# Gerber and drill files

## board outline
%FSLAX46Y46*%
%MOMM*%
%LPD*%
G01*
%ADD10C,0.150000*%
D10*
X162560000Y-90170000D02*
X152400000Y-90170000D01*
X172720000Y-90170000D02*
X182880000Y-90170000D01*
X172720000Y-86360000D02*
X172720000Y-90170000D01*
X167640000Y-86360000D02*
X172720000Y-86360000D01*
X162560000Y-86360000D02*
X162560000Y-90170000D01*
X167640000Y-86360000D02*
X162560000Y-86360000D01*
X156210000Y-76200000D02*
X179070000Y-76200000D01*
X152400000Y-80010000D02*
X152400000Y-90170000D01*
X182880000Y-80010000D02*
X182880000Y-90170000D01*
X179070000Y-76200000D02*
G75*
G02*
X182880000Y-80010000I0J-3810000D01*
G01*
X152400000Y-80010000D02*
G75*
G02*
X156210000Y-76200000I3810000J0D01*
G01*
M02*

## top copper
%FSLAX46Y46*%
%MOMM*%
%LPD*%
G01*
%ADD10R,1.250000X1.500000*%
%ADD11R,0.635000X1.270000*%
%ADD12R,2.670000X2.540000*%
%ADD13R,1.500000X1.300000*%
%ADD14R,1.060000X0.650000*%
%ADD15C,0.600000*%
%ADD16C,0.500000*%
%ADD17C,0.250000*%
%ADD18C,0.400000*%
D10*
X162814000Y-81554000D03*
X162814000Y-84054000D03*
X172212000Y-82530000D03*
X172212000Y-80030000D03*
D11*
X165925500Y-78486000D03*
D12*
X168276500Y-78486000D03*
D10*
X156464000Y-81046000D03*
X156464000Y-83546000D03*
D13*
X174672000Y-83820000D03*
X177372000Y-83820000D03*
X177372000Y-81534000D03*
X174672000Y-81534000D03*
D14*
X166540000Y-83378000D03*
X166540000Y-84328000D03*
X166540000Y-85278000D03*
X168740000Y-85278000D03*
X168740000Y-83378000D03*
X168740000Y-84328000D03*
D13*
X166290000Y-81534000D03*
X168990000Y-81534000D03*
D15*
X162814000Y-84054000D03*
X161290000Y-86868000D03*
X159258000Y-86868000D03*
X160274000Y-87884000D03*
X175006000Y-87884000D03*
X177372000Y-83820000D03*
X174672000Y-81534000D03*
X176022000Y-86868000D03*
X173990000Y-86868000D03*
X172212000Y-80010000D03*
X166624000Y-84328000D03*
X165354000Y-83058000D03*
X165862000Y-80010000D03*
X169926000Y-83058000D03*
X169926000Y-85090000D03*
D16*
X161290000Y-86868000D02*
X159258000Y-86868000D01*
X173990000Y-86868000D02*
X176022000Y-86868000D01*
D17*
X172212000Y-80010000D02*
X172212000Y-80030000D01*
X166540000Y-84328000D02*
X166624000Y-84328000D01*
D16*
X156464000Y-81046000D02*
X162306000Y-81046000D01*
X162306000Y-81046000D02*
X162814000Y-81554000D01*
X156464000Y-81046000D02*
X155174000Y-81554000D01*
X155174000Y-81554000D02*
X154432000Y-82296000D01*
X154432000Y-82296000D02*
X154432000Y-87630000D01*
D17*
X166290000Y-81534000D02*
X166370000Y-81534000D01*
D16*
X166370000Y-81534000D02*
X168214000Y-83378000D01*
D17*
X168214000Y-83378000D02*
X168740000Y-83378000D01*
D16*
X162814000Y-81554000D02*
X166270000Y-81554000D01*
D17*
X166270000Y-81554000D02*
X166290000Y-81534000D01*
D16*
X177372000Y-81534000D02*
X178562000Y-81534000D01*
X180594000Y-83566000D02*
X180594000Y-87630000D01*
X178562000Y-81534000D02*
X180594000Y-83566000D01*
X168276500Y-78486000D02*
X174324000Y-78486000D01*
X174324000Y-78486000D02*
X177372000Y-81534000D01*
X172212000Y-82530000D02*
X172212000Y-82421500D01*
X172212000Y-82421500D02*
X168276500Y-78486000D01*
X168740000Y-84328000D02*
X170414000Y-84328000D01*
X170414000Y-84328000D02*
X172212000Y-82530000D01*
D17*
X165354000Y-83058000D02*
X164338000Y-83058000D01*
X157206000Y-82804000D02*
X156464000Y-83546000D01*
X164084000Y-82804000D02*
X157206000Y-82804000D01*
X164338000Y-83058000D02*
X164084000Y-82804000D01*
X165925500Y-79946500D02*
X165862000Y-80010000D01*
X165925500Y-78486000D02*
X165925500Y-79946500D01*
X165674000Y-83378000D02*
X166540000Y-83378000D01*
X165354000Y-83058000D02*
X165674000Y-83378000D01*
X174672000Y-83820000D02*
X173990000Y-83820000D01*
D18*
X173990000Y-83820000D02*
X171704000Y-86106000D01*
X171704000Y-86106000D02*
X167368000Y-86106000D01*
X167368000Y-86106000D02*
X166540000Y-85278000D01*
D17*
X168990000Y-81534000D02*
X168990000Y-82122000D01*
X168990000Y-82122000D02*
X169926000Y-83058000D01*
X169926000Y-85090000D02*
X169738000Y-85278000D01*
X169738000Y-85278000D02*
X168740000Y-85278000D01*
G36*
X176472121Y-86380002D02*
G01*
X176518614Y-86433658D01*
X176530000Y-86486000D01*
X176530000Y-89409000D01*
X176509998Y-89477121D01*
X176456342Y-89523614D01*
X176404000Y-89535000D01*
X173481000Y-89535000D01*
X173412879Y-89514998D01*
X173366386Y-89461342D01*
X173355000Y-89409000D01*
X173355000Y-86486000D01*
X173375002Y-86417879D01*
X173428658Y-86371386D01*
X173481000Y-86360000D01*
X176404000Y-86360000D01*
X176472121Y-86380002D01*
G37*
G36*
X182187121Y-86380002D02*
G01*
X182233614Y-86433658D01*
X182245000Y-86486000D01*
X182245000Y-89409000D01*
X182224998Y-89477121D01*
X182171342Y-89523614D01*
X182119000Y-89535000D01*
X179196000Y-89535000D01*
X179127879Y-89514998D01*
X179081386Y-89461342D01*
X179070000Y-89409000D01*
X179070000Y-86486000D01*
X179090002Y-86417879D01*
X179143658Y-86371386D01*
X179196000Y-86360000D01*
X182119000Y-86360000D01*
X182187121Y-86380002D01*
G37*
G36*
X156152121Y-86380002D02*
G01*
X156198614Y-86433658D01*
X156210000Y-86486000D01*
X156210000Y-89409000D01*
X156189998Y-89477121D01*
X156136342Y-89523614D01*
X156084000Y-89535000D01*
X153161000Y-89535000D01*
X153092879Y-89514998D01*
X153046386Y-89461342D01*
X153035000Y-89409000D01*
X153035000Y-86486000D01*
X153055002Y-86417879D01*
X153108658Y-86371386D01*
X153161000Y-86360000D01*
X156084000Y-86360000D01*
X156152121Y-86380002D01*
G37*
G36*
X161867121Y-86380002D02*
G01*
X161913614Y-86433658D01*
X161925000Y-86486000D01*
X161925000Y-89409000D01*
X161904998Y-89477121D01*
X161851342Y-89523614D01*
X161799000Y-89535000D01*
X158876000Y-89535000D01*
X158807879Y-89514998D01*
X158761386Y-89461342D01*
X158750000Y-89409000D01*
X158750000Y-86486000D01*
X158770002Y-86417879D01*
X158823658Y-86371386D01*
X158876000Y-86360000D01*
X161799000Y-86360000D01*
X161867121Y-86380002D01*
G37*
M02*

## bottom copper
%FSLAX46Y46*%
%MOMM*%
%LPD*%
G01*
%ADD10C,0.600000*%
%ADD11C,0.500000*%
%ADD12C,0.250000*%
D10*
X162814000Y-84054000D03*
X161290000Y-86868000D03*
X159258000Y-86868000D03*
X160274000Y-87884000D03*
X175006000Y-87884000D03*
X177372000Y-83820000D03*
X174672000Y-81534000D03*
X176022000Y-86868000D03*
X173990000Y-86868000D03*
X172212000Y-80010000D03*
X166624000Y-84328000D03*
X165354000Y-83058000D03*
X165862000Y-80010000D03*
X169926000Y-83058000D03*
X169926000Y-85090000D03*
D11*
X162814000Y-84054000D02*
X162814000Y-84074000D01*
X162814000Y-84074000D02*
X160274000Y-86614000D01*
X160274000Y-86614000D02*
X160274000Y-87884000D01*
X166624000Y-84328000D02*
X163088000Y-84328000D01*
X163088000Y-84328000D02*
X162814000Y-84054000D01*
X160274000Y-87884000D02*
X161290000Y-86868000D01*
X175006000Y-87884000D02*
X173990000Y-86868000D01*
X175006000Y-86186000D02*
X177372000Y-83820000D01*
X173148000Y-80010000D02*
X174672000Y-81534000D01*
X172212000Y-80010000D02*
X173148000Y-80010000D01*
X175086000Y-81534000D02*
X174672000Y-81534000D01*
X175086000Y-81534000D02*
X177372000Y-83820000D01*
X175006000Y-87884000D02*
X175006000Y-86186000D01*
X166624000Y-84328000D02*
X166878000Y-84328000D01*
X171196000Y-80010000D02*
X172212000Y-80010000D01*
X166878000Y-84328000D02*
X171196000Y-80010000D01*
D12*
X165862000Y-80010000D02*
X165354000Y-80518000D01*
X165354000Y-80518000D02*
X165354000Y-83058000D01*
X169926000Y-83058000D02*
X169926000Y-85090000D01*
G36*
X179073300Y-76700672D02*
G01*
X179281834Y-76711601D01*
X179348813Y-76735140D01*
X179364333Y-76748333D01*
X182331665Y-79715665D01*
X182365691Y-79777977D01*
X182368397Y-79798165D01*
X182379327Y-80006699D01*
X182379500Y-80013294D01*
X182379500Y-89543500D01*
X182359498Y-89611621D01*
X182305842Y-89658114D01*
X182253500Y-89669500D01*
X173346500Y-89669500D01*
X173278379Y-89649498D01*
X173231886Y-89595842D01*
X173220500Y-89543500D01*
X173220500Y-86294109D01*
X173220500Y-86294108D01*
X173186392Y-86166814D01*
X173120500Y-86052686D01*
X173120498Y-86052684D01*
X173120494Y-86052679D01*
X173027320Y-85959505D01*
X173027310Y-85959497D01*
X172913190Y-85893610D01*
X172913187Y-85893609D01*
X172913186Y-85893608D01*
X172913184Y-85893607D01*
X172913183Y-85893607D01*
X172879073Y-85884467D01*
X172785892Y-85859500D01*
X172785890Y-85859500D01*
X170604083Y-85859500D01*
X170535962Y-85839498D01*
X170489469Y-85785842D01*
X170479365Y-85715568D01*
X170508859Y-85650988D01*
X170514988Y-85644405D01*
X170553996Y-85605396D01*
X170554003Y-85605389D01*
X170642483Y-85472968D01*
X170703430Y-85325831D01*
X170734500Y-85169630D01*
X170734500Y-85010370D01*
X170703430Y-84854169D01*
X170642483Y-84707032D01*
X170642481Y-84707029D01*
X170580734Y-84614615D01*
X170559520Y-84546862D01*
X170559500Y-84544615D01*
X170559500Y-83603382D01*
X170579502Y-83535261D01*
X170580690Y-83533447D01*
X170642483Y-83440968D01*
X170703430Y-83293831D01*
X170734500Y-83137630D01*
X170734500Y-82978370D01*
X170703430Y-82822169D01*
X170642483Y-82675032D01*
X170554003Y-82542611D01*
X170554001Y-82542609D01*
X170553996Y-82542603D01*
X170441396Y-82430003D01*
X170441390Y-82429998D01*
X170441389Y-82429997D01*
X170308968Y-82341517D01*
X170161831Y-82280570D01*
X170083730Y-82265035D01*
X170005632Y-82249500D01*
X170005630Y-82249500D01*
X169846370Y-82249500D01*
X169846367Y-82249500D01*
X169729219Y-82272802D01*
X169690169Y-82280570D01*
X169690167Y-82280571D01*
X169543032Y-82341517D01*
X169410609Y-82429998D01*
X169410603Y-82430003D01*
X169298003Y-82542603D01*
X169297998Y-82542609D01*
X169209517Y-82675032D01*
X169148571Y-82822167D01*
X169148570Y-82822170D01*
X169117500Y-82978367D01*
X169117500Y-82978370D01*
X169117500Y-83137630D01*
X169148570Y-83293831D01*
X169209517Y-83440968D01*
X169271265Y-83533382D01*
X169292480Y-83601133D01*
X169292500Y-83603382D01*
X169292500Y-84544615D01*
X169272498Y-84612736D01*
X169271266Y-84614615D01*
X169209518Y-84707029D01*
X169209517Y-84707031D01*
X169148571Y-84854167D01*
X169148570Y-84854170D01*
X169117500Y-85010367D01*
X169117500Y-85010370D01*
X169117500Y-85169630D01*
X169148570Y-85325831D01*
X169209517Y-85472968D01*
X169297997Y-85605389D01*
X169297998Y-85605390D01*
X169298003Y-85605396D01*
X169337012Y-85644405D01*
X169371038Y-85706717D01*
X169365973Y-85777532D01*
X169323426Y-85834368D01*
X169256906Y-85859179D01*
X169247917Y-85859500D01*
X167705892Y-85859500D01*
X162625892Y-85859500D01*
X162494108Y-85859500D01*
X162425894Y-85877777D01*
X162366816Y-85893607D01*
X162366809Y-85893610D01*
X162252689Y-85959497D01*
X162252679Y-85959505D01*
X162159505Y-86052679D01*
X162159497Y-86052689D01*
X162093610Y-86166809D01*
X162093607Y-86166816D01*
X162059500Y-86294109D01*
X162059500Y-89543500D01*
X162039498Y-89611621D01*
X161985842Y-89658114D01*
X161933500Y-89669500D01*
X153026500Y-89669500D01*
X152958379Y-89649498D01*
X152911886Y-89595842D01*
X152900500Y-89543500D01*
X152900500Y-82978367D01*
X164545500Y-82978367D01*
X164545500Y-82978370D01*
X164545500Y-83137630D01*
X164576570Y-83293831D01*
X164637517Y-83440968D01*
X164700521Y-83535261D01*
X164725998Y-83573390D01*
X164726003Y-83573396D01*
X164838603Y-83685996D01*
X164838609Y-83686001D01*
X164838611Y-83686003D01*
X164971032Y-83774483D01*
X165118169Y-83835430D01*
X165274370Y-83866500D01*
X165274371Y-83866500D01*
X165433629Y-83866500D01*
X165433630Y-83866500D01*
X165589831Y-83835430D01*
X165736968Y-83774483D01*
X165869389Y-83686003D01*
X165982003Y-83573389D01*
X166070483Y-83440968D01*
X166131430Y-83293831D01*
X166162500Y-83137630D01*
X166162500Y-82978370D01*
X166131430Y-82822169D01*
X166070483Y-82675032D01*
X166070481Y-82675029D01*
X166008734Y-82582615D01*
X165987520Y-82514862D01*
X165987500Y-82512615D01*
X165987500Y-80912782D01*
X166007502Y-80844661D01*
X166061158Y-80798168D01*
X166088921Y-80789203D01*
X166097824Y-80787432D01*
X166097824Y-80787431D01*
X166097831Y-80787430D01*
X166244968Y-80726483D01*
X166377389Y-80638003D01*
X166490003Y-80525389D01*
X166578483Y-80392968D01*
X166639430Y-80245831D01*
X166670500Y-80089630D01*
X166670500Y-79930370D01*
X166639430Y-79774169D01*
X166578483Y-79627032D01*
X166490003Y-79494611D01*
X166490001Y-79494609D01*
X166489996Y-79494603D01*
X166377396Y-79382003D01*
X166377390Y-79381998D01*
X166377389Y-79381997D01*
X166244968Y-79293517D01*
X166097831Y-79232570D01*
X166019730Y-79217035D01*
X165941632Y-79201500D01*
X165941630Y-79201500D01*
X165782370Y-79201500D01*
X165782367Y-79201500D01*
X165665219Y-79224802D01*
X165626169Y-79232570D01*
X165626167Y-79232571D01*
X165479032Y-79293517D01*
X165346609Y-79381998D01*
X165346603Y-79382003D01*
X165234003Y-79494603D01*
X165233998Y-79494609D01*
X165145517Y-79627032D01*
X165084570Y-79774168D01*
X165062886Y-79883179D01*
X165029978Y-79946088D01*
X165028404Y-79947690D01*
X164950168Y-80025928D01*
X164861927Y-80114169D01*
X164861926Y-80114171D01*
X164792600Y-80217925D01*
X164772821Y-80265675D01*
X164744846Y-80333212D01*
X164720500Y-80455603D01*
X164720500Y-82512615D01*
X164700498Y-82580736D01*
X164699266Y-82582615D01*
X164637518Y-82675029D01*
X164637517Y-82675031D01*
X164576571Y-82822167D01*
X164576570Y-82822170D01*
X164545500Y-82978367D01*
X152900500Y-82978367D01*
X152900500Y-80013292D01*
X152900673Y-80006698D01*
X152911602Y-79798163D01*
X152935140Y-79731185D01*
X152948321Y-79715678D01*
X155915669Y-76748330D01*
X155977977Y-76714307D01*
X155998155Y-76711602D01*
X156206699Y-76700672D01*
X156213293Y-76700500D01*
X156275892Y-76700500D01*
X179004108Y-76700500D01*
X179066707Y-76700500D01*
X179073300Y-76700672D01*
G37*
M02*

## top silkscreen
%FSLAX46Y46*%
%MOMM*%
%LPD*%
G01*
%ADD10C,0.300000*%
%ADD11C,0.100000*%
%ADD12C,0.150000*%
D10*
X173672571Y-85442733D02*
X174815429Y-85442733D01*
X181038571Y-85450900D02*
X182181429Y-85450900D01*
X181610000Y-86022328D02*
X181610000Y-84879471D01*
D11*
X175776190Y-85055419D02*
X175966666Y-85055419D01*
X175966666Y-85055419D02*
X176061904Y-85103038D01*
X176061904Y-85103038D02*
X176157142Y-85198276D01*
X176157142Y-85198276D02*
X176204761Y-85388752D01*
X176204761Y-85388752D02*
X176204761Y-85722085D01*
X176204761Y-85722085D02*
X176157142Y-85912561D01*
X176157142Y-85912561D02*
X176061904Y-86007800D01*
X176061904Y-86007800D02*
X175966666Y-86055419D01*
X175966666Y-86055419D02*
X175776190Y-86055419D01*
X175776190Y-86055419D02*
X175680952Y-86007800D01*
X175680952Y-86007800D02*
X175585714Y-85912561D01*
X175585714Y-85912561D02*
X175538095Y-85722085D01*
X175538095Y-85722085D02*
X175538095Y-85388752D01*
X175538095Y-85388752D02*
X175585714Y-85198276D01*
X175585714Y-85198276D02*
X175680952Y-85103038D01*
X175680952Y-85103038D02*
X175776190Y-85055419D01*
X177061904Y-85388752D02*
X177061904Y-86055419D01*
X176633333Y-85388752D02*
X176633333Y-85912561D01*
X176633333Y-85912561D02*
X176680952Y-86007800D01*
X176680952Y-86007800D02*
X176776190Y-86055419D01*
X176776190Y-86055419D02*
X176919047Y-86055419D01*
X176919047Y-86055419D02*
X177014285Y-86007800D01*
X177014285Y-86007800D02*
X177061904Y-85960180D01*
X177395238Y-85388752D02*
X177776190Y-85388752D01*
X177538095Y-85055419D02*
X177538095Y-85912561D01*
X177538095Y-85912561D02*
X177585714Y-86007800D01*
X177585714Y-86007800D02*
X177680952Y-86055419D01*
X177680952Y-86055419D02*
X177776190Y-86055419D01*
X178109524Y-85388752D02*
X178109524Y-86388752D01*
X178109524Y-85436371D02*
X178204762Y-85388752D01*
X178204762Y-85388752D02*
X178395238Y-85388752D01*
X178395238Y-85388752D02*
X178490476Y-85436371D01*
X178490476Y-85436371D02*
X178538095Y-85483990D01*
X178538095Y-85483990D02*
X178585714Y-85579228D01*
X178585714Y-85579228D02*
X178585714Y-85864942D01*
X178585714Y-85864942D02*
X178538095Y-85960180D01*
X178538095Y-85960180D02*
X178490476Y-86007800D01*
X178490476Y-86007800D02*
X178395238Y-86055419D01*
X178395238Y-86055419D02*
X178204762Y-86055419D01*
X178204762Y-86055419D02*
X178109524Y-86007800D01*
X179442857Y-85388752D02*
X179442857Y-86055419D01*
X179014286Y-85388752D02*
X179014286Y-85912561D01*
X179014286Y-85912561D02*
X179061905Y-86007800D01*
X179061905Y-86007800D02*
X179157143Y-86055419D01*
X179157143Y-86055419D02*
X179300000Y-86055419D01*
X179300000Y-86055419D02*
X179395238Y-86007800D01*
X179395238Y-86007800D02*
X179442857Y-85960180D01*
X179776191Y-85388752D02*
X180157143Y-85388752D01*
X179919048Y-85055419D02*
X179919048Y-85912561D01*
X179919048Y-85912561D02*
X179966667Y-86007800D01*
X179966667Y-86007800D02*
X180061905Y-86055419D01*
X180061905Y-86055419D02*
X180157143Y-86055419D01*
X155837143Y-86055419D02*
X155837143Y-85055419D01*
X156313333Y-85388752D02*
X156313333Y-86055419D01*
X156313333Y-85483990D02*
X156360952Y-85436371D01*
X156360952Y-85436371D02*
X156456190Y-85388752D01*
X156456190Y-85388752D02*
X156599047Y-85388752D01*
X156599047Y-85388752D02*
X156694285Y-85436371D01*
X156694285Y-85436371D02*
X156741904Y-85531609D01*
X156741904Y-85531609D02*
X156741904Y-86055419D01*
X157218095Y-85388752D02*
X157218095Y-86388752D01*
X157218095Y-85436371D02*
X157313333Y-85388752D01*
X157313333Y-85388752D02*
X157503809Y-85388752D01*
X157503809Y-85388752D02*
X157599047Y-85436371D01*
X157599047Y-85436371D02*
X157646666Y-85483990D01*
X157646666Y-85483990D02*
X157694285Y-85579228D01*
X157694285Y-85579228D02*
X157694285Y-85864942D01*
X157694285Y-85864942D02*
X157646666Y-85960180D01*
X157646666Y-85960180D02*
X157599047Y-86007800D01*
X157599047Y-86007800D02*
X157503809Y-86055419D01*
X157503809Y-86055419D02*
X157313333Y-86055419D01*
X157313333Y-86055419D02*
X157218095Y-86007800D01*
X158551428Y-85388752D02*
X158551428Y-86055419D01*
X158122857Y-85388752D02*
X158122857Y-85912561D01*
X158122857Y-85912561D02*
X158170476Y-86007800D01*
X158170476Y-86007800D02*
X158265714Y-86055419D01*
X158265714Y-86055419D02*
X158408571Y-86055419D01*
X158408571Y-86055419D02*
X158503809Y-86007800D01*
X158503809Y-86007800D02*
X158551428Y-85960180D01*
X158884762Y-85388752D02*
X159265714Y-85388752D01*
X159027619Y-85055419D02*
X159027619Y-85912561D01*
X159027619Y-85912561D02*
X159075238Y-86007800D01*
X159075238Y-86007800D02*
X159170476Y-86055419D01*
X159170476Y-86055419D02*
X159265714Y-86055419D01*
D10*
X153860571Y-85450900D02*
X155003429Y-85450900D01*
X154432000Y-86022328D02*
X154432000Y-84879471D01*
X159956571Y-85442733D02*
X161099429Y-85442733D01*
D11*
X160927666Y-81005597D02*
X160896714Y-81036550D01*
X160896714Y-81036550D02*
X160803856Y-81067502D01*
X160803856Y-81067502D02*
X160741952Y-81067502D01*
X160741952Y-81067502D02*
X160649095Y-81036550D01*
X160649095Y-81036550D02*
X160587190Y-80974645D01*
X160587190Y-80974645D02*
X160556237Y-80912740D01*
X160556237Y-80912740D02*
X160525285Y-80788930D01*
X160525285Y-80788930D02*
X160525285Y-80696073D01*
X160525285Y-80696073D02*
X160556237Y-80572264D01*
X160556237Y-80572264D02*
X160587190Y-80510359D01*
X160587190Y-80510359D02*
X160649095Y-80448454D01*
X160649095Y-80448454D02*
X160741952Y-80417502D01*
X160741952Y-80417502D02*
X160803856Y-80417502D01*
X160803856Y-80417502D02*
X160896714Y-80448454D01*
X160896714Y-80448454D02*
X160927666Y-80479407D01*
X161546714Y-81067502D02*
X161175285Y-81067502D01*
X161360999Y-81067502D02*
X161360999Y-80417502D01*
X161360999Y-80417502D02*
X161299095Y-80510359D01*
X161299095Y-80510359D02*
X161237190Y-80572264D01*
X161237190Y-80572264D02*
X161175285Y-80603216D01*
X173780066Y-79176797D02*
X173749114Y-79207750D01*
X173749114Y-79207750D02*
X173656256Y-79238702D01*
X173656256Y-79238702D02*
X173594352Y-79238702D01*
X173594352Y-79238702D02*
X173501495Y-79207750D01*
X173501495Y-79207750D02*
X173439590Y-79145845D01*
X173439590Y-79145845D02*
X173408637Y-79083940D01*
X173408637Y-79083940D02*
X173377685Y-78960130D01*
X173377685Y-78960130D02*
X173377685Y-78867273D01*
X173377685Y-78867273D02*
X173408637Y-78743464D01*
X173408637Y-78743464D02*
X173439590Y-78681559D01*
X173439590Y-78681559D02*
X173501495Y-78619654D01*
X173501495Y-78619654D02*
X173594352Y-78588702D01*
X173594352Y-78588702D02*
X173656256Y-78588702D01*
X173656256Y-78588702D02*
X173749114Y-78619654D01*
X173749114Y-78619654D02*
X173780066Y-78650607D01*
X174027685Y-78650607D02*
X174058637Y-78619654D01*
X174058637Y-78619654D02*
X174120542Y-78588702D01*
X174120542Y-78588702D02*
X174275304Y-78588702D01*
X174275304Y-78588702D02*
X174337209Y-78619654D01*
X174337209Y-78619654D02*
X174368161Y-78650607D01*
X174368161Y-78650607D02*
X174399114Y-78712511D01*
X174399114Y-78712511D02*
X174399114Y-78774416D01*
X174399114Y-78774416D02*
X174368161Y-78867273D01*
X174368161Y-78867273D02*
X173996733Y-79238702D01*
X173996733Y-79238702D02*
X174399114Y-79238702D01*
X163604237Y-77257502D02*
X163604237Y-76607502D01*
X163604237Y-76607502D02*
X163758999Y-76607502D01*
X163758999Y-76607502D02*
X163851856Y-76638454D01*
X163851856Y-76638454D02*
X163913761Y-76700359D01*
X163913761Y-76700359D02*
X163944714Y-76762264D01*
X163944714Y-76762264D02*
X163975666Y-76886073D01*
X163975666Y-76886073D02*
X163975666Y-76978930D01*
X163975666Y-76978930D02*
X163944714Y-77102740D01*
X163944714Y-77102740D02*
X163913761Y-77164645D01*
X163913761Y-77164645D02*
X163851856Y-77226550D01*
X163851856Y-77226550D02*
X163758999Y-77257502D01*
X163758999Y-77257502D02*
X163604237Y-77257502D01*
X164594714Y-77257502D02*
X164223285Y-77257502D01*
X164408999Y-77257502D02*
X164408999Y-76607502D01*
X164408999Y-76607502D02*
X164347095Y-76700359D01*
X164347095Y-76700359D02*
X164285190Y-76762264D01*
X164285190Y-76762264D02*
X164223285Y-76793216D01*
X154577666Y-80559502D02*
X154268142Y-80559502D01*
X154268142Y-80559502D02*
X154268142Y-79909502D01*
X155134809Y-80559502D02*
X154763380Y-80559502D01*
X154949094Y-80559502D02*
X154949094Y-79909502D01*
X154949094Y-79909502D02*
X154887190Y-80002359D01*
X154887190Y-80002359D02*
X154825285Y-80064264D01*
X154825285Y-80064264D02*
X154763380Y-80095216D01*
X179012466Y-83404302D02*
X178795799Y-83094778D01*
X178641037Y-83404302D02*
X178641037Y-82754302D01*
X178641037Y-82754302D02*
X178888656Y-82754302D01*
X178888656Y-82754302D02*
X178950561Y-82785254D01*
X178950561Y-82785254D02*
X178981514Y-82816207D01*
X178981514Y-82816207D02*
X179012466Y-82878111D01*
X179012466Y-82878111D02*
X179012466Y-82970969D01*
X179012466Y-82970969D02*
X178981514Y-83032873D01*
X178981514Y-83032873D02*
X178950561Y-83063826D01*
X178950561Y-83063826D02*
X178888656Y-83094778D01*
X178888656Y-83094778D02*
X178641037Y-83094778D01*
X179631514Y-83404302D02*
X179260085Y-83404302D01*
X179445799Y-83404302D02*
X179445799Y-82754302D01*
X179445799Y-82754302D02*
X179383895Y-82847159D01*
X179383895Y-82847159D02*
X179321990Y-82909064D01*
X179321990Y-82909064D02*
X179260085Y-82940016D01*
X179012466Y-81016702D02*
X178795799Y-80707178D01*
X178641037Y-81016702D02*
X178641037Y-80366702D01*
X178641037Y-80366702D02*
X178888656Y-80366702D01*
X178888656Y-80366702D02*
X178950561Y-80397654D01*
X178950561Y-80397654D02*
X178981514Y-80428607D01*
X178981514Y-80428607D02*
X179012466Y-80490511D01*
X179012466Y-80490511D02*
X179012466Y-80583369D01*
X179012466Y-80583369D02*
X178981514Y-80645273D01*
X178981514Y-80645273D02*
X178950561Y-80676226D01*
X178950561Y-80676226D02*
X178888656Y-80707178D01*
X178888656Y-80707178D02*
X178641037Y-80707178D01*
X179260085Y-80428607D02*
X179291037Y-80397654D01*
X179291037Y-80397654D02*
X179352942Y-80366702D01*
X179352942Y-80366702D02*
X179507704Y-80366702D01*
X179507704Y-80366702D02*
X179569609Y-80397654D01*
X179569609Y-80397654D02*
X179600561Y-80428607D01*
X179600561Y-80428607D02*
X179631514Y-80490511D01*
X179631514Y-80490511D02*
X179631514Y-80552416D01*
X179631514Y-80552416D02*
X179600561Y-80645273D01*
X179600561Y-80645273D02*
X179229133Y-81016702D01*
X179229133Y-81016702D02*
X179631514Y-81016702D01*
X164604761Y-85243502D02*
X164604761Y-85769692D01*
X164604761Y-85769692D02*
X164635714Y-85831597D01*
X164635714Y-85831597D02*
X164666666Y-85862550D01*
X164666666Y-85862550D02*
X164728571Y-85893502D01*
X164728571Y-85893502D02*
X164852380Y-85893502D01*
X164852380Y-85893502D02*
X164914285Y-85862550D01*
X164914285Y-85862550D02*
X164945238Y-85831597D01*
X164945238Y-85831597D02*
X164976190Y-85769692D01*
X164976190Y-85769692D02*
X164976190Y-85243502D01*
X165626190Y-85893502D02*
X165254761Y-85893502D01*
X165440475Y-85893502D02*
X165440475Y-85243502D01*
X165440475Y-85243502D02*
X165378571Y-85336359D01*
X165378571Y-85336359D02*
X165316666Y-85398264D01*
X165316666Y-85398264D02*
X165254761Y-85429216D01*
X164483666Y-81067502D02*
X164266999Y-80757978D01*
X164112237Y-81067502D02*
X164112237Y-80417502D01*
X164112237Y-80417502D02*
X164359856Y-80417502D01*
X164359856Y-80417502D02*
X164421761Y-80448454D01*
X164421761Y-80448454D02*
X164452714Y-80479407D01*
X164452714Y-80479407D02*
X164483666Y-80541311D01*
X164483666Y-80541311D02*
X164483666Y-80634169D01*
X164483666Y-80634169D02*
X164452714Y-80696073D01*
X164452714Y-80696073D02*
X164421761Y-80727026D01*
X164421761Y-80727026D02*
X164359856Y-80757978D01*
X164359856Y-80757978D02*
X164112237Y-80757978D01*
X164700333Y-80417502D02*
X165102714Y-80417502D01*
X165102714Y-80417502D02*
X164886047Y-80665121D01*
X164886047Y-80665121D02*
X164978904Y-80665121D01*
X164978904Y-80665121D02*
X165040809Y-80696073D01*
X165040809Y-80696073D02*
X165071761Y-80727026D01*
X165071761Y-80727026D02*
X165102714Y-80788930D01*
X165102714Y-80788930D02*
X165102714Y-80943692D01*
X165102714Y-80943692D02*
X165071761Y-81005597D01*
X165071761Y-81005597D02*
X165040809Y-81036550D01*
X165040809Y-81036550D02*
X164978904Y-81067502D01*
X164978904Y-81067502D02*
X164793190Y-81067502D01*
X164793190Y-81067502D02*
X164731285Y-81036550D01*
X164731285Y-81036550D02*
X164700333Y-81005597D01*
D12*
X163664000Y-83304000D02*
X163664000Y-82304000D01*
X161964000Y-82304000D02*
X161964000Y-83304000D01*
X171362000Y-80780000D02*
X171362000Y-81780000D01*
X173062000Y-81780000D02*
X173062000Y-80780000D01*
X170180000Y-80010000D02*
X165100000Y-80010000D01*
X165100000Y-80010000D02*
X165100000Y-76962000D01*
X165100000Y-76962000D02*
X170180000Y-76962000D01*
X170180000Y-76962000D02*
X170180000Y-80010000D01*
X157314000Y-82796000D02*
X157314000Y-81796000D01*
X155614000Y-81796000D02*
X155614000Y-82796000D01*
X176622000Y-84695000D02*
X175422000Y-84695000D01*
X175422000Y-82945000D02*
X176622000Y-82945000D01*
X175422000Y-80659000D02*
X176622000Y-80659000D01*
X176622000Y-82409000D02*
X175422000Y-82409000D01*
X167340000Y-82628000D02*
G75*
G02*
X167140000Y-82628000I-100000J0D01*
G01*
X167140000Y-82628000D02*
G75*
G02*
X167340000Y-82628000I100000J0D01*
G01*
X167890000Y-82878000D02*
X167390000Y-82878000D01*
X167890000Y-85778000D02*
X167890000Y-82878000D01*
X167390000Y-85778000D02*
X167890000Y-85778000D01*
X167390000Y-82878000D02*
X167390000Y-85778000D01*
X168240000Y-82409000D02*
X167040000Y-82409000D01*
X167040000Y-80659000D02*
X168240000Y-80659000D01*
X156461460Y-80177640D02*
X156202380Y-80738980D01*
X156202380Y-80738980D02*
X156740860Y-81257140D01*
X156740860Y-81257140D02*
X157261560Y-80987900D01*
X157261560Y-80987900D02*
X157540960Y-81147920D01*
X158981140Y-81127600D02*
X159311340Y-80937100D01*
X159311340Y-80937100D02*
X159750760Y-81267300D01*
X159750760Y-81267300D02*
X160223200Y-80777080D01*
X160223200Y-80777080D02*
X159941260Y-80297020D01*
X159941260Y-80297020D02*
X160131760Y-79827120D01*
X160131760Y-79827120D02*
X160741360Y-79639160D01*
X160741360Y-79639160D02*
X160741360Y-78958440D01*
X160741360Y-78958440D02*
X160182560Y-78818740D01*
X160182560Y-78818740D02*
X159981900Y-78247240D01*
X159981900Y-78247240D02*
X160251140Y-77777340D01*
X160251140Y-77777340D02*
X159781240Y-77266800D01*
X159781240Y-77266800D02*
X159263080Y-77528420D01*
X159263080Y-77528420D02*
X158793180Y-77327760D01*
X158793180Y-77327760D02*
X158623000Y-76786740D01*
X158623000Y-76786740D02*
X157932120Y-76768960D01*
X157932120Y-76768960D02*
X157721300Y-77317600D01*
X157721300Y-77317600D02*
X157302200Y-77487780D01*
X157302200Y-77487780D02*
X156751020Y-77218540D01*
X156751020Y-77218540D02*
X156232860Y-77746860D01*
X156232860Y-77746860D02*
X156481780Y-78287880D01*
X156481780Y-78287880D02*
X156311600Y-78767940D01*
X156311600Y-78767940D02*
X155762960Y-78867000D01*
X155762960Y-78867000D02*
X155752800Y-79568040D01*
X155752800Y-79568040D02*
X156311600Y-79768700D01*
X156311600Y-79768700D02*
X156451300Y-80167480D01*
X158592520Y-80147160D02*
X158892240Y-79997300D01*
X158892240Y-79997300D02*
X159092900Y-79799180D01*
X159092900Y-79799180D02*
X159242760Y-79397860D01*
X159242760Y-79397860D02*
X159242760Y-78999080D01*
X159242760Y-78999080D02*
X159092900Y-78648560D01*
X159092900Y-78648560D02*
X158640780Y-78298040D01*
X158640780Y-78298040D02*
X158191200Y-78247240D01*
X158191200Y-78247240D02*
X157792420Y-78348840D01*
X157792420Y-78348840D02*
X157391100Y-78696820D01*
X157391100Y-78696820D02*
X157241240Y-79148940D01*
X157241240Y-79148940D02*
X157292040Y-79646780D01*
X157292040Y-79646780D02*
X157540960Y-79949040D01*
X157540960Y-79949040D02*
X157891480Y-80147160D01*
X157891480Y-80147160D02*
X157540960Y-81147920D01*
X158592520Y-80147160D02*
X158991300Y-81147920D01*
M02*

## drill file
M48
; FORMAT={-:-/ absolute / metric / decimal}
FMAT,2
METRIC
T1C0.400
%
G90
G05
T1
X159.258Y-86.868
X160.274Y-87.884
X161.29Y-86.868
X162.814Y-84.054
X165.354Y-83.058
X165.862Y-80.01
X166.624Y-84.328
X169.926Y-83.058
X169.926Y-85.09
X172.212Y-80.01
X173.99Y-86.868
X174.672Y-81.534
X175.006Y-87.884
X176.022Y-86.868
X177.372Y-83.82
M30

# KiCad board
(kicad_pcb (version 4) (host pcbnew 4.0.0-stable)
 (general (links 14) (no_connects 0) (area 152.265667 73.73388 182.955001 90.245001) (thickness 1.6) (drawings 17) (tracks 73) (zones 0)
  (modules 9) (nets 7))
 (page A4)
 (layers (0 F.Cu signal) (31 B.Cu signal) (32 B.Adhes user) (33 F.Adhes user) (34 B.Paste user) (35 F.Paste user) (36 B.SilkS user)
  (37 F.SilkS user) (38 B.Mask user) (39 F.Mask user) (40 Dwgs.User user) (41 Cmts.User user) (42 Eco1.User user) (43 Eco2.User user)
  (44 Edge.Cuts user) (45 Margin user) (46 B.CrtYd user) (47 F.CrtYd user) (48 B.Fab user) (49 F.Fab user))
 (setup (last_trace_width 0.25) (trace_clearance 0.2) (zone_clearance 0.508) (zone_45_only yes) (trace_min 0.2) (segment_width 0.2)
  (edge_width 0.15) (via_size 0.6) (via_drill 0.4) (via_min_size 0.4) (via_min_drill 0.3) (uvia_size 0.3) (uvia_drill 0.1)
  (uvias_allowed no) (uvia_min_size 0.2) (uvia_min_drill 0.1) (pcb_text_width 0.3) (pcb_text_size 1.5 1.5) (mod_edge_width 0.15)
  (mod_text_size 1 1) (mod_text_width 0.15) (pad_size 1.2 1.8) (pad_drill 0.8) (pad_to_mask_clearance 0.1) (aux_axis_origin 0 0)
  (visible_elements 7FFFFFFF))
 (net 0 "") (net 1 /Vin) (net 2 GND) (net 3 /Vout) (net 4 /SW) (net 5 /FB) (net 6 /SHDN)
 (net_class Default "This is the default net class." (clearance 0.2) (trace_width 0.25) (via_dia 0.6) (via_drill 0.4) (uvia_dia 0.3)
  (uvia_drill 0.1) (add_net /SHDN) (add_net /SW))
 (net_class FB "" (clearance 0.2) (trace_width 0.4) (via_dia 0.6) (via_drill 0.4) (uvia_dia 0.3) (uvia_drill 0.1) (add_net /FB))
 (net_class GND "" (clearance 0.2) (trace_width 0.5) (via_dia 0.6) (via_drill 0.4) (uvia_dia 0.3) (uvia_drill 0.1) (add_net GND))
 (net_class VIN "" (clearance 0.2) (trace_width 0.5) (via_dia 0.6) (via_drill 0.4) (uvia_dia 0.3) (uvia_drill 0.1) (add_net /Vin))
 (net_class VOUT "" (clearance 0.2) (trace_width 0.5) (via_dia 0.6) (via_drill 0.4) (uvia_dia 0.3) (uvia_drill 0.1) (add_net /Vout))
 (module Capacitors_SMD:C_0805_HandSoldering (layer F.Cu) (at 162.814 82.804 270)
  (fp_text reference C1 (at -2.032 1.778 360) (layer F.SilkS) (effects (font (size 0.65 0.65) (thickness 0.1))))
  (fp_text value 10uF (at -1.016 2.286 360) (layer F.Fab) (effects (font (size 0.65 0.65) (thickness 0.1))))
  (fp_line (start 0.5 -0.85) (end -0.5 -0.85) (layer F.SilkS) (width 0.15))
  (fp_line (start -0.5 0.85) (end 0.5 0.85) (layer F.SilkS) (width 0.15))
  (pad 1 smd rect (at -1.25 0 270) (size 1.5 1.25) (layers F.Cu F.Paste F.Mask) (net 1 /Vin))
  (pad 2 smd rect (at 1.25 0 270) (size 1.5 1.25) (layers F.Cu F.Paste F.Mask) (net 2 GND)))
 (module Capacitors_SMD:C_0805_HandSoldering (layer F.Cu) (at 172.212 81.28 90)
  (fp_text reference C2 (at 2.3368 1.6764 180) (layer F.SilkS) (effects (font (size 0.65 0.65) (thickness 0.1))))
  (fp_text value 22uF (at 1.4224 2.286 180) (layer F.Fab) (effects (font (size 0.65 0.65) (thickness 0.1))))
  (fp_line (start 0.5 -0.85) (end -0.5 -0.85) (layer F.SilkS) (width 0.15))
  (fp_line (start -0.5 0.85) (end 0.5 0.85) (layer F.SilkS) (width 0.15))
  (pad 1 smd rect (at -1.25 0 90) (size 1.5 1.25) (layers F.Cu F.Paste F.Mask) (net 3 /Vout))
  (pad 2 smd rect (at 1.25 0 90) (size 1.5 1.25) (layers F.Cu F.Paste F.Mask) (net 2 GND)))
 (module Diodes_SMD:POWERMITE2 (layer F.Cu) (at 167.64 78.486 180)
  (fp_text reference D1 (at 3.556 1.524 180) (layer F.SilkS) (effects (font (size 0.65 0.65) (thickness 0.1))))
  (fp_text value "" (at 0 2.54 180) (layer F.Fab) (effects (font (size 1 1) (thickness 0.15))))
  (fp_line (start -2.54 -1.524) (end 2.54 -1.524) (layer F.SilkS) (width 0.15))
  (fp_line (start 2.54 -1.524) (end 2.54 1.524) (layer F.SilkS) (width 0.15))
  (fp_line (start 2.54 1.524) (end -2.54 1.524) (layer F.SilkS) (width 0.15))
  (fp_line (start -2.54 1.524) (end -2.54 -1.524) (layer F.SilkS) (width 0.15))
  (pad 2 smd rect (at 1.7145 0) (size 0.635 1.27) (layers F.Cu F.Paste F.Mask) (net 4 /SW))
  (pad 1 smd rect (at -0.6365 0) (size 2.67 2.54) (layers F.Cu F.Paste F.Mask) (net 3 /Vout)))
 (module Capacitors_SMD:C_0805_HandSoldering (layer F.Cu) (at 156.464 82.296 270)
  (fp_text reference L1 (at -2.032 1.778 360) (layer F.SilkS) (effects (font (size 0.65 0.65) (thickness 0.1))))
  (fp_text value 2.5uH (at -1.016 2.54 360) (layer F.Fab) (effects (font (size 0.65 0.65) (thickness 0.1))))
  (fp_line (start 0.5 -0.85) (end -0.5 -0.85) (layer F.SilkS) (width 0.15))
  (fp_line (start -0.5 0.85) (end 0.5 0.85) (layer F.SilkS) (width 0.15))
  (pad 1 smd rect (at -1.25 0 270) (size 1.5 1.25) (layers F.Cu F.Paste F.Mask) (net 1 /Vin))
  (pad 2 smd rect (at 1.25 0 270) (size 1.5 1.25) (layers F.Cu F.Paste F.Mask) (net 4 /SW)))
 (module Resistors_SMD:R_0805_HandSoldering (layer F.Cu) (at 176.022 83.82)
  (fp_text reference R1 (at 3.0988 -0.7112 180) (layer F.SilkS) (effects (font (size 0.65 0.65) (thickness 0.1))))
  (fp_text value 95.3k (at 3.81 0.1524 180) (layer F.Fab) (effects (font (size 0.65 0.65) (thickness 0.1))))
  (fp_line (start 0.6 0.875) (end -0.6 0.875) (layer F.SilkS) (width 0.15))
  (fp_line (start -0.6 -0.875) (end 0.6 -0.875) (layer F.SilkS) (width 0.15))
  (pad 1 smd rect (at -1.35 0) (size 1.5 1.3) (layers F.Cu F.Paste F.Mask) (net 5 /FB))
  (pad 2 smd rect (at 1.35 0) (size 1.5 1.3) (layers F.Cu F.Paste F.Mask) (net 2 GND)))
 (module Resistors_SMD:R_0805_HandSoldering (layer F.Cu) (at 176.022 81.534 180)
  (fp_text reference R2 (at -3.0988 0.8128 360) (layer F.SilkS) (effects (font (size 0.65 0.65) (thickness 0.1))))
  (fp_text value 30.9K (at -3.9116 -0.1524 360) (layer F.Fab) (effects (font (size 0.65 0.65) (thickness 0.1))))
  (fp_line (start 0.6 0.875) (end -0.6 0.875) (layer F.SilkS) (width 0.15))
  (fp_line (start -0.6 -0.875) (end 0.6 -0.875) (layer F.SilkS) (width 0.15))
  (pad 1 smd rect (at -1.35 0 180) (size 1.5 1.3) (layers F.Cu F.Paste F.Mask) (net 3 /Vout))
  (pad 2 smd rect (at 1.35 0 180) (size 1.5 1.3) (layers F.Cu F.Paste F.Mask) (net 2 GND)))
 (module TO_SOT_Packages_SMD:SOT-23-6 (layer F.Cu) (at 167.64 84.328)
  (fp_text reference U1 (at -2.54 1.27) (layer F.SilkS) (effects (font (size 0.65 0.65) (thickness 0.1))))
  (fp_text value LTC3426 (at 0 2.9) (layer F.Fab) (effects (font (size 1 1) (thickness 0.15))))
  (fp_circle (center -0.4 -1.7) (end -0.3 -1.7) (layer F.SilkS) (width 0.15))
  (fp_line (start 0.25 -1.45) (end -0.25 -1.45) (layer F.SilkS) (width 0.15))
  (fp_line (start 0.25 1.45) (end 0.25 -1.45) (layer F.SilkS) (width 0.15))
  (fp_line (start -0.25 1.45) (end 0.25 1.45) (layer F.SilkS) (width 0.15))
  (fp_line (start -0.25 -1.45) (end -0.25 1.45) (layer F.SilkS) (width 0.15))
  (pad 1 smd rect (at -1.1 -0.95) (size 1.06 0.65) (layers F.Cu F.Paste F.Mask) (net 4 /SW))
  (pad 2 smd rect (at -1.1 0) (size 1.06 0.65) (layers F.Cu F.Paste F.Mask) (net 2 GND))
  (pad 3 smd rect (at -1.1 0.95) (size 1.06 0.65) (layers F.Cu F.Paste F.Mask) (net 5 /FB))
  (pad 4 smd rect (at 1.1 0.95) (size 1.06 0.65) (layers F.Cu F.Paste F.Mask) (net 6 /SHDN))
  (pad 6 smd rect (at 1.1 -0.95) (size 1.06 0.65) (layers F.Cu F.Paste F.Mask) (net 1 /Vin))
  (pad 5 smd rect (at 1.1 0) (size 1.06 0.65) (layers F.Cu F.Paste F.Mask) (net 3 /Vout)))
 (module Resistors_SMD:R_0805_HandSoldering (layer F.Cu) (at 167.64 81.534)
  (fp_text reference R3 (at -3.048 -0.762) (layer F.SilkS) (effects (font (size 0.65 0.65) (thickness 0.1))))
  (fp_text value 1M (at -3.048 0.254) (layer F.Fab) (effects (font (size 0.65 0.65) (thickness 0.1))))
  (fp_line (start 0.6 0.875) (end -0.6 0.875) (layer F.SilkS) (width 0.15))
  (fp_line (start -0.6 -0.875) (end 0.6 -0.875) (layer F.SilkS) (width 0.15))
  (pad 1 smd rect (at -1.35 0) (size 1.5 1.3) (layers F.Cu F.Paste F.Mask) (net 1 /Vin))
  (pad 2 smd rect (at 1.35 0) (size 1.5 1.3) (layers F.Cu F.Paste F.Mask) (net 6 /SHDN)))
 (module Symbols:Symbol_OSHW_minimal (layer F.Cu) (at 158.242 79.248)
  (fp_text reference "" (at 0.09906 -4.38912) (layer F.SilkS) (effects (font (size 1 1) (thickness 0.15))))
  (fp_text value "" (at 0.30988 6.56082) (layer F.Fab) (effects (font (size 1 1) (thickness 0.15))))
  (fp_line (start -1.78054 0.92964) (end -2.03962 1.49098) (layer F.SilkS) (width 0.15))
  (fp_line (start -2.03962 1.49098) (end -1.50114 2.00914) (layer F.SilkS) (width 0.15))
  (fp_line (start -1.50114 2.00914) (end -0.98044 1.7399) (layer F.SilkS) (width 0.15))
  (fp_line (start -0.98044 1.7399) (end -0.70104 1.89992) (layer F.SilkS) (width 0.15))
  (fp_line (start 0.73914 1.8796) (end 1.06934 1.6891) (layer F.SilkS) (width 0.15))
  (fp_line (start 1.06934 1.6891) (end 1.50876 2.0193) (layer F.SilkS) (width 0.15))
  (fp_line (start 1.50876 2.0193) (end 1.9812 1.52908) (layer F.SilkS) (width 0.15))
  (fp_line (start 1.9812 1.52908) (end 1.69926 1.04902) (layer F.SilkS) (width 0.15))
  (fp_line (start 1.69926 1.04902) (end 1.88976 0.57912) (layer F.SilkS) (width 0.15))
  (fp_line (start 1.88976 0.57912) (end 2.49936 0.39116) (layer F.SilkS) (width 0.15))
  (fp_line (start 2.49936 0.39116) (end 2.49936 -0.28956) (layer F.SilkS) (width 0.15))
  (fp_line (start 2.49936 -0.28956) (end 1.94056 -0.42926) (layer F.SilkS) (width 0.15))
  (fp_line (start 1.94056 -0.42926) (end 1.7399 -1.00076) (layer F.SilkS) (width 0.15))
  (fp_line (start 1.7399 -1.00076) (end 2.00914 -1.47066) (layer F.SilkS) (width 0.15))
  (fp_line (start 2.00914 -1.47066) (end 1.53924 -1.9812) (layer F.SilkS) (width 0.15))
  (fp_line (start 1.53924 -1.9812) (end 1.02108 -1.71958) (layer F.SilkS) (width 0.15))
  (fp_line (start 1.02108 -1.71958) (end 0.55118 -1.92024) (layer F.SilkS) (width 0.15))
  (fp_line (start 0.55118 -1.92024) (end 0.381 -2.46126) (layer F.SilkS) (width 0.15))
  (fp_line (start 0.381 -2.46126) (end -0.30988 -2.47904) (layer F.SilkS) (width 0.15))
  (fp_line (start -0.30988 -2.47904) (end -0.5207 -1.9304) (layer F.SilkS) (width 0.15))
  (fp_line (start -0.5207 -1.9304) (end -0.9398 -1.76022) (layer F.SilkS) (width 0.15))
  (fp_line (start -0.9398 -1.76022) (end -1.49098 -2.02946) (layer F.SilkS) (width 0.15))
  (fp_line (start -1.49098 -2.02946) (end -2.00914 -1.50114) (layer F.SilkS) (width 0.15))
  (fp_line (start -2.00914 -1.50114) (end -1.76022 -0.96012) (layer F.SilkS) (width 0.15))
  (fp_line (start -1.76022 -0.96012) (end -1.9304 -0.48006) (layer F.SilkS) (width 0.15))
  (fp_line (start -1.9304 -0.48006) (end -2.47904 -0.381) (layer F.SilkS) (width 0.15))
  (fp_line (start -2.47904 -0.381) (end -2.4892 0.32004) (layer F.SilkS) (width 0.15))
  (fp_line (start -2.4892 0.32004) (end -1.9304 0.5207) (layer F.SilkS) (width 0.15))
  (fp_line (start -1.9304 0.5207) (end -1.7907 0.91948) (layer F.SilkS) (width 0.15))
  (fp_line (start 0.35052 0.89916) (end 0.65024 0.7493) (layer F.SilkS) (width 0.15))
  (fp_line (start 0.65024 0.7493) (end 0.8509 0.55118) (layer F.SilkS) (width 0.15))
  (fp_line (start 0.8509 0.55118) (end 1.00076 0.14986) (layer F.SilkS) (width 0.15))
  (fp_line (start 1.00076 0.14986) (end 1.00076 -0.24892) (layer F.SilkS) (width 0.15))
  (fp_line (start 1.00076 -0.24892) (end 0.8509 -0.59944) (layer F.SilkS) (width 0.15))
  (fp_line (start 0.8509 -0.59944) (end 0.39878 -0.94996) (layer F.SilkS) (width 0.15))
  (fp_line (start 0.39878 -0.94996) (end -0.0508 -1.00076) (layer F.SilkS) (width 0.15))
  (fp_line (start -0.0508 -1.00076) (end -0.44958 -0.89916) (layer F.SilkS) (width 0.15))
  (fp_line (start -0.44958 -0.89916) (end -0.8509 -0.55118) (layer F.SilkS) (width 0.15))
  (fp_line (start -0.8509 -0.55118) (end -1.00076 -0.09906) (layer F.SilkS) (width 0.15))
  (fp_line (start -1.00076 -0.09906) (end -0.94996 0.39878) (layer F.SilkS) (width 0.15))
  (fp_line (start -0.94996 0.39878) (end -0.70104 0.70104) (layer F.SilkS) (width 0.15))
  (fp_line (start -0.70104 0.70104) (end -0.35052 0.89916) (layer F.SilkS) (width 0.15))
  (fp_line (start -0.35052 0.89916) (end -0.70104 1.89992) (layer F.SilkS) (width 0.15))
  (fp_line (start 0.35052 0.89916) (end 0.7493 1.89992) (layer F.SilkS) (width 0.15)))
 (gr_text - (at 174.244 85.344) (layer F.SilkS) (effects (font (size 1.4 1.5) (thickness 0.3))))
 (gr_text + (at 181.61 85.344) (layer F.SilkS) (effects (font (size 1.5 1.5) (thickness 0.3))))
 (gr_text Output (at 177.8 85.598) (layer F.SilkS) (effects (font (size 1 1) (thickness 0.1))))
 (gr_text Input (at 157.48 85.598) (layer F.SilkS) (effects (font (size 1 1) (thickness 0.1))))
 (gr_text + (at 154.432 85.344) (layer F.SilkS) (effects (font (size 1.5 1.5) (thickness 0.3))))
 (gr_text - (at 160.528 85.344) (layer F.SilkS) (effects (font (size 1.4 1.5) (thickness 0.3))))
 (gr_line (start 162.56 90.17) (end 152.4 90.17) (angle 90) (layer Edge.Cuts) (width 0.15))
 (gr_line (start 172.72 90.17) (end 182.88 90.17) (angle 90) (layer Edge.Cuts) (width 0.15))
 (gr_line (start 172.72 86.36) (end 172.72 90.17) (angle 90) (layer Edge.Cuts) (width 0.15))
 (gr_line (start 167.64 86.36) (end 172.72 86.36) (angle 90) (layer Edge.Cuts) (width 0.15))
 (gr_line (start 162.56 86.36) (end 162.56 90.17) (angle 90) (layer Edge.Cuts) (width 0.15))
 (gr_line (start 167.64 86.36) (end 162.56 86.36) (angle 90) (layer Edge.Cuts) (width 0.15))
 (gr_line (start 156.21 76.2) (end 179.07 76.2) (angle 90) (layer Edge.Cuts) (width 0.15))
 (gr_line (start 152.4 80.01) (end 152.4 90.17) (angle 90) (layer Edge.Cuts) (width 0.15))
 (gr_line (start 182.88 80.01) (end 182.88 90.17) (angle 90) (layer Edge.Cuts) (width 0.15))
 (gr_arc (start 179.07 80.01) (end 179.07 76.2) (angle 90) (layer Edge.Cuts) (width 0.15))
 (gr_arc (start 156.21 80.01) (end 152.4 80.01) (angle 90) (layer Edge.Cuts) (width 0.15))
 (via (at 162.814 84.054) (size 0.6) (drill 0.4) (layers F.Cu B.Cu) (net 2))
 (via (at 161.29 86.868) (size 0.6) (drill 0.4) (layers F.Cu B.Cu) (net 2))
 (segment (start 161.29 86.868) (end 159.258 86.868) (width 0.5) (layer F.Cu) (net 2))
 (via (at 159.258 86.868) (size 0.6) (drill 0.4) (layers F.Cu B.Cu) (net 2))
 (segment (start 162.814 84.054) (end 162.814 84.074) (width 0.5) (layer B.Cu) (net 2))
 (segment (start 162.814 84.074) (end 160.274 86.614) (width 0.5) (layer B.Cu) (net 2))
 (segment (start 160.274 86.614) (end 160.274 87.884) (width 0.5) (layer B.Cu) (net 2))
 (via (at 160.274 87.884) (size 0.6) (drill 0.4) (layers F.Cu B.Cu) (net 2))
 (segment (start 166.624 84.328) (end 163.088 84.328) (width 0.5) (layer B.Cu) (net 2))
 (segment (start 163.088 84.328) (end 162.814 84.054) (width 0.5) (layer B.Cu) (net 2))
 (segment (start 160.274 87.884) (end 161.29 86.868) (width 0.5) (layer B.Cu) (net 2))
 (segment (start 175.006 87.884) (end 173.99 86.868) (width 0.5) (layer B.Cu) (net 2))
 (segment (start 175.006 86.186) (end 177.372 83.82) (width 0.5) (layer B.Cu) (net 2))
 (via (at 175.006 87.884) (size 0.6) (drill 0.4) (layers F.Cu B.Cu) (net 2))
 (via (at 177.372 83.82) (size 0.6) (drill 0.4) (layers F.Cu B.Cu) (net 2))
 (segment (start 173.148 80.01) (end 174.672 81.534) (width 0.5) (layer B.Cu) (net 2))
 (segment (start 172.212 80.01) (end 173.148 80.01) (width 0.5) (layer B.Cu) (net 2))
 (via (at 174.672 81.534) (size 0.6) (drill 0.4) (layers F.Cu B.Cu) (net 2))
 (segment (start 175.086 81.534) (end 174.672 81.534) (width 0.5) (layer B.Cu) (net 2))
 (segment (start 175.086 81.534) (end 177.372 83.82) (width 0.5) (layer B.Cu) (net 2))
 (segment (start 175.006 87.884) (end 175.006 86.186) (width 0.5) (layer B.Cu) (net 2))
 (via (at 176.022 86.868) (size 0.6) (drill 0.4) (layers F.Cu B.Cu) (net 2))
 (segment (start 173.99 86.868) (end 176.022 86.868) (width 0.5) (layer F.Cu) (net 2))
 (via (at 173.99 86.868) (size 0.6) (drill 0.4) (layers F.Cu B.Cu) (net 2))
 (segment (start 166.624 84.328) (end 166.878 84.328) (width 0.5) (layer B.Cu) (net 2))
 (segment (start 171.196 80.01) (end 172.212 80.01) (width 0.5) (layer B.Cu) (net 2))
 (segment (start 166.878 84.328) (end 171.196 80.01) (width 0.5) (layer B.Cu) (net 2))
 (segment (start 172.212 80.01) (end 172.212 80.03) (width 0.25) (layer F.Cu) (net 2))
 (via (at 172.212 80.01) (size 0.6) (drill 0.4) (layers F.Cu B.Cu) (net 2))
 (segment (start 166.54 84.328) (end 166.624 84.328) (width 0.25) (layer F.Cu) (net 2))
 (via (at 166.624 84.328) (size 0.6) (drill 0.4) (layers F.Cu B.Cu) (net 2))
 (segment (start 156.464 81.046) (end 162.306 81.046) (width 0.5) (layer F.Cu) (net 1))
 (segment (start 162.306 81.046) (end 162.814 81.554) (width 0.5) (layer F.Cu) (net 1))
 (segment (start 156.464 81.046) (end 155.174 81.554) (width 0.5) (layer F.Cu) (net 1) (status 10))
 (segment (start 155.174 81.554) (end 154.432 82.296) (width 0.5) (layer F.Cu) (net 1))
 (segment (start 154.432 82.296) (end 154.432 87.63) (width 0.5) (layer F.Cu) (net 1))
 (segment (start 166.29 81.534) (end 166.37 81.534) (width 0.25) (layer F.Cu) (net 1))
 (segment (start 166.37 81.534) (end 168.214 83.378) (width 0.5) (layer F.Cu) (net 1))
 (segment (start 168.214 83.378) (end 168.74 83.378) (width 0.25) (layer F.Cu) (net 1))
 (segment (start 162.814 81.554) (end 166.27 81.554) (width 0.5) (layer F.Cu) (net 1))
 (segment (start 166.27 81.554) (end 166.29 81.534) (width 0.25) (layer F.Cu) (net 1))
 (segment (start 177.372 81.534) (end 178.562 81.534) (width 0.5) (layer F.Cu) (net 3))
 (segment (start 180.594 83.566) (end 180.594 87.63) (width 0.5) (layer F.Cu) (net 3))
 (segment (start 178.562 81.534) (end 180.594 83.566) (width 0.5) (layer F.Cu) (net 3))
 (segment (start 168.2765 78.486) (end 174.324 78.486) (width 0.5) (layer F.Cu) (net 3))
 (segment (start 174.324 78.486) (end 177.372 81.534) (width 0.5) (layer F.Cu) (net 3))
 (segment (start 172.212 82.53) (end 172.212 82.4215) (width 0.5) (layer F.Cu) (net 3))
 (segment (start 172.212 82.4215) (end 168.2765 78.486) (width 0.5) (layer F.Cu) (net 3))
 (segment (start 168.74 84.328) (end 170.414 84.328) (width 0.5) (layer F.Cu) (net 3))
 (segment (start 170.414 84.328) (end 172.212 82.53) (width 0.5) (layer F.Cu) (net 3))
 (segment (start 165.354 83.058) (end 164.338 83.058) (width 0.25) (layer F.Cu) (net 4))
 (segment (start 157.206 82.804) (end 156.464 83.546) (width 0.25) (layer F.Cu) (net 4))
 (segment (start 164.084 82.804) (end 157.206 82.804) (width 0.25) (layer F.Cu) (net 4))
 (segment (start 164.338 83.058) (end 164.084 82.804) (width 0.25) (layer F.Cu) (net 4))
 (via (at 165.354 83.058) (size 0.6) (drill 0.4) (layers F.Cu B.Cu) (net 4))
 (segment (start 165.9255 79.9465) (end 165.862 80.01) (width 0.25) (layer F.Cu) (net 4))
 (via (at 165.862 80.01) (size 0.6) (drill 0.4) (layers F.Cu B.Cu) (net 4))
 (segment (start 165.862 80.01) (end 165.354 80.518) (width 0.25) (layer B.Cu) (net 4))
 (segment (start 165.354 80.518) (end 165.354 83.058) (width 0.25) (layer B.Cu) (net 4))
 (segment (start 165.9255 78.486) (end 165.9255 79.9465) (width 0.25) (layer F.Cu) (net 4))
 (segment (start 165.674 83.378) (end 166.54 83.378) (width 0.25) (layer F.Cu) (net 4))
 (segment (start 165.354 83.058) (end 165.674 83.378) (width 0.25) (layer F.Cu) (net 4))
 (segment (start 174.672 83.82) (end 173.99 83.82) (width 0.25) (layer F.Cu) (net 5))
 (segment (start 173.99 83.82) (end 171.704 86.106) (width 0.4) (layer F.Cu) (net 5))
 (segment (start 171.704 86.106) (end 167.368 86.106) (width 0.4) (layer F.Cu) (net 5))
 (segment (start 167.368 86.106) (end 166.54 85.278) (width 0.4) (layer F.Cu) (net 5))
 (segment (start 168.99 81.534) (end 168.99 82.122) (width 0.25) (layer F.Cu) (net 6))
 (segment (start 168.99 82.122) (end 169.926 83.058) (width 0.25) (layer F.Cu) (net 6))
 (via (at 169.926 83.058) (size 0.6) (drill 0.4) (layers F.Cu B.Cu) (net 6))
 (segment (start 169.926 83.058) (end 169.926 85.09) (width 0.25) (layer B.Cu) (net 6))
 (via (at 169.926 85.09) (size 0.6) (drill 0.4) (layers F.Cu B.Cu) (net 6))
 (segment (start 169.926 85.09) (end 169.738 85.278) (width 0.25) (layer F.Cu) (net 6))
 (segment (start 169.738 85.278) (end 168.74 85.278) (width 0.25) (layer F.Cu) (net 6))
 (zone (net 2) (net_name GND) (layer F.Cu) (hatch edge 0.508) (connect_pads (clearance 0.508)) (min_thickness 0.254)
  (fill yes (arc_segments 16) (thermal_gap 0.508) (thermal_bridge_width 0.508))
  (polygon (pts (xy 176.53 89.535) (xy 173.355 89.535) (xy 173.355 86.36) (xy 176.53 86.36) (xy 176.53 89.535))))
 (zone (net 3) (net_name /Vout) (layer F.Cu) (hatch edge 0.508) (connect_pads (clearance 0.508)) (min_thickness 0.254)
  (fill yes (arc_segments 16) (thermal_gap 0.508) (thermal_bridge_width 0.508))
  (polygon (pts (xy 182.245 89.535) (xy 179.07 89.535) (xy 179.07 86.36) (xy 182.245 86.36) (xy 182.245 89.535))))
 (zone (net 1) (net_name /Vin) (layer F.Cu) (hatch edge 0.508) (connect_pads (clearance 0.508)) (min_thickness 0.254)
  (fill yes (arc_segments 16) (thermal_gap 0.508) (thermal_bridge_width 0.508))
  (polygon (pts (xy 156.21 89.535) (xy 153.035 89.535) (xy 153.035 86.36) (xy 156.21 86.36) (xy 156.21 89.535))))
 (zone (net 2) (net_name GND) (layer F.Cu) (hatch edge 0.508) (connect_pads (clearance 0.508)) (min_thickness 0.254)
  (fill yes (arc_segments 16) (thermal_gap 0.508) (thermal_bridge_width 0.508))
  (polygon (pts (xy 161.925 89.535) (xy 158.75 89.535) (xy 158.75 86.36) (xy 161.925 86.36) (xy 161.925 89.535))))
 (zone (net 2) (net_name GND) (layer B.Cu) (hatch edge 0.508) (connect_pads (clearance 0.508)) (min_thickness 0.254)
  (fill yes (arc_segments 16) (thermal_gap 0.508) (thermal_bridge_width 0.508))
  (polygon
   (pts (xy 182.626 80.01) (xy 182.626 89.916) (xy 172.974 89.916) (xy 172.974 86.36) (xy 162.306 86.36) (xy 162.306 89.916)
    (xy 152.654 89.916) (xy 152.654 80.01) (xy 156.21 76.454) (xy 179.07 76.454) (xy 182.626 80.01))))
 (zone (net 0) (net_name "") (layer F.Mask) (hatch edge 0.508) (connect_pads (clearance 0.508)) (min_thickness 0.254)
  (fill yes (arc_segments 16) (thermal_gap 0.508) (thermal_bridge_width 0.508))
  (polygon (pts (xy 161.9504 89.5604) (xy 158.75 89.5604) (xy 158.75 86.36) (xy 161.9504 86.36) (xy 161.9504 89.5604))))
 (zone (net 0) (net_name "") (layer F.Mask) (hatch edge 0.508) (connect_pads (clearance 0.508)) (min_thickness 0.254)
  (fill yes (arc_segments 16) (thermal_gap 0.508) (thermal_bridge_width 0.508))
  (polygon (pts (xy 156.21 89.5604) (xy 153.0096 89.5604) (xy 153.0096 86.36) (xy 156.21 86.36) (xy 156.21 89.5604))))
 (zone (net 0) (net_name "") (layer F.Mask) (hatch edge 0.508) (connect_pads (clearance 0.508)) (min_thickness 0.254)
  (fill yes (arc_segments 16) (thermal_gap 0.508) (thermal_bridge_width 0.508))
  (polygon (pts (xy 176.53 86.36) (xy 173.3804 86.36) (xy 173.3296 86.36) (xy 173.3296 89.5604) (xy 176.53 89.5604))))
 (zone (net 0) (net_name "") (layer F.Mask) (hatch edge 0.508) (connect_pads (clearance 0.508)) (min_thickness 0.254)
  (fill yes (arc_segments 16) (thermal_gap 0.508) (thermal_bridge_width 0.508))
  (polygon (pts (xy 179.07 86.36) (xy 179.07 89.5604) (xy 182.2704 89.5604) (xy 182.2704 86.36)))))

